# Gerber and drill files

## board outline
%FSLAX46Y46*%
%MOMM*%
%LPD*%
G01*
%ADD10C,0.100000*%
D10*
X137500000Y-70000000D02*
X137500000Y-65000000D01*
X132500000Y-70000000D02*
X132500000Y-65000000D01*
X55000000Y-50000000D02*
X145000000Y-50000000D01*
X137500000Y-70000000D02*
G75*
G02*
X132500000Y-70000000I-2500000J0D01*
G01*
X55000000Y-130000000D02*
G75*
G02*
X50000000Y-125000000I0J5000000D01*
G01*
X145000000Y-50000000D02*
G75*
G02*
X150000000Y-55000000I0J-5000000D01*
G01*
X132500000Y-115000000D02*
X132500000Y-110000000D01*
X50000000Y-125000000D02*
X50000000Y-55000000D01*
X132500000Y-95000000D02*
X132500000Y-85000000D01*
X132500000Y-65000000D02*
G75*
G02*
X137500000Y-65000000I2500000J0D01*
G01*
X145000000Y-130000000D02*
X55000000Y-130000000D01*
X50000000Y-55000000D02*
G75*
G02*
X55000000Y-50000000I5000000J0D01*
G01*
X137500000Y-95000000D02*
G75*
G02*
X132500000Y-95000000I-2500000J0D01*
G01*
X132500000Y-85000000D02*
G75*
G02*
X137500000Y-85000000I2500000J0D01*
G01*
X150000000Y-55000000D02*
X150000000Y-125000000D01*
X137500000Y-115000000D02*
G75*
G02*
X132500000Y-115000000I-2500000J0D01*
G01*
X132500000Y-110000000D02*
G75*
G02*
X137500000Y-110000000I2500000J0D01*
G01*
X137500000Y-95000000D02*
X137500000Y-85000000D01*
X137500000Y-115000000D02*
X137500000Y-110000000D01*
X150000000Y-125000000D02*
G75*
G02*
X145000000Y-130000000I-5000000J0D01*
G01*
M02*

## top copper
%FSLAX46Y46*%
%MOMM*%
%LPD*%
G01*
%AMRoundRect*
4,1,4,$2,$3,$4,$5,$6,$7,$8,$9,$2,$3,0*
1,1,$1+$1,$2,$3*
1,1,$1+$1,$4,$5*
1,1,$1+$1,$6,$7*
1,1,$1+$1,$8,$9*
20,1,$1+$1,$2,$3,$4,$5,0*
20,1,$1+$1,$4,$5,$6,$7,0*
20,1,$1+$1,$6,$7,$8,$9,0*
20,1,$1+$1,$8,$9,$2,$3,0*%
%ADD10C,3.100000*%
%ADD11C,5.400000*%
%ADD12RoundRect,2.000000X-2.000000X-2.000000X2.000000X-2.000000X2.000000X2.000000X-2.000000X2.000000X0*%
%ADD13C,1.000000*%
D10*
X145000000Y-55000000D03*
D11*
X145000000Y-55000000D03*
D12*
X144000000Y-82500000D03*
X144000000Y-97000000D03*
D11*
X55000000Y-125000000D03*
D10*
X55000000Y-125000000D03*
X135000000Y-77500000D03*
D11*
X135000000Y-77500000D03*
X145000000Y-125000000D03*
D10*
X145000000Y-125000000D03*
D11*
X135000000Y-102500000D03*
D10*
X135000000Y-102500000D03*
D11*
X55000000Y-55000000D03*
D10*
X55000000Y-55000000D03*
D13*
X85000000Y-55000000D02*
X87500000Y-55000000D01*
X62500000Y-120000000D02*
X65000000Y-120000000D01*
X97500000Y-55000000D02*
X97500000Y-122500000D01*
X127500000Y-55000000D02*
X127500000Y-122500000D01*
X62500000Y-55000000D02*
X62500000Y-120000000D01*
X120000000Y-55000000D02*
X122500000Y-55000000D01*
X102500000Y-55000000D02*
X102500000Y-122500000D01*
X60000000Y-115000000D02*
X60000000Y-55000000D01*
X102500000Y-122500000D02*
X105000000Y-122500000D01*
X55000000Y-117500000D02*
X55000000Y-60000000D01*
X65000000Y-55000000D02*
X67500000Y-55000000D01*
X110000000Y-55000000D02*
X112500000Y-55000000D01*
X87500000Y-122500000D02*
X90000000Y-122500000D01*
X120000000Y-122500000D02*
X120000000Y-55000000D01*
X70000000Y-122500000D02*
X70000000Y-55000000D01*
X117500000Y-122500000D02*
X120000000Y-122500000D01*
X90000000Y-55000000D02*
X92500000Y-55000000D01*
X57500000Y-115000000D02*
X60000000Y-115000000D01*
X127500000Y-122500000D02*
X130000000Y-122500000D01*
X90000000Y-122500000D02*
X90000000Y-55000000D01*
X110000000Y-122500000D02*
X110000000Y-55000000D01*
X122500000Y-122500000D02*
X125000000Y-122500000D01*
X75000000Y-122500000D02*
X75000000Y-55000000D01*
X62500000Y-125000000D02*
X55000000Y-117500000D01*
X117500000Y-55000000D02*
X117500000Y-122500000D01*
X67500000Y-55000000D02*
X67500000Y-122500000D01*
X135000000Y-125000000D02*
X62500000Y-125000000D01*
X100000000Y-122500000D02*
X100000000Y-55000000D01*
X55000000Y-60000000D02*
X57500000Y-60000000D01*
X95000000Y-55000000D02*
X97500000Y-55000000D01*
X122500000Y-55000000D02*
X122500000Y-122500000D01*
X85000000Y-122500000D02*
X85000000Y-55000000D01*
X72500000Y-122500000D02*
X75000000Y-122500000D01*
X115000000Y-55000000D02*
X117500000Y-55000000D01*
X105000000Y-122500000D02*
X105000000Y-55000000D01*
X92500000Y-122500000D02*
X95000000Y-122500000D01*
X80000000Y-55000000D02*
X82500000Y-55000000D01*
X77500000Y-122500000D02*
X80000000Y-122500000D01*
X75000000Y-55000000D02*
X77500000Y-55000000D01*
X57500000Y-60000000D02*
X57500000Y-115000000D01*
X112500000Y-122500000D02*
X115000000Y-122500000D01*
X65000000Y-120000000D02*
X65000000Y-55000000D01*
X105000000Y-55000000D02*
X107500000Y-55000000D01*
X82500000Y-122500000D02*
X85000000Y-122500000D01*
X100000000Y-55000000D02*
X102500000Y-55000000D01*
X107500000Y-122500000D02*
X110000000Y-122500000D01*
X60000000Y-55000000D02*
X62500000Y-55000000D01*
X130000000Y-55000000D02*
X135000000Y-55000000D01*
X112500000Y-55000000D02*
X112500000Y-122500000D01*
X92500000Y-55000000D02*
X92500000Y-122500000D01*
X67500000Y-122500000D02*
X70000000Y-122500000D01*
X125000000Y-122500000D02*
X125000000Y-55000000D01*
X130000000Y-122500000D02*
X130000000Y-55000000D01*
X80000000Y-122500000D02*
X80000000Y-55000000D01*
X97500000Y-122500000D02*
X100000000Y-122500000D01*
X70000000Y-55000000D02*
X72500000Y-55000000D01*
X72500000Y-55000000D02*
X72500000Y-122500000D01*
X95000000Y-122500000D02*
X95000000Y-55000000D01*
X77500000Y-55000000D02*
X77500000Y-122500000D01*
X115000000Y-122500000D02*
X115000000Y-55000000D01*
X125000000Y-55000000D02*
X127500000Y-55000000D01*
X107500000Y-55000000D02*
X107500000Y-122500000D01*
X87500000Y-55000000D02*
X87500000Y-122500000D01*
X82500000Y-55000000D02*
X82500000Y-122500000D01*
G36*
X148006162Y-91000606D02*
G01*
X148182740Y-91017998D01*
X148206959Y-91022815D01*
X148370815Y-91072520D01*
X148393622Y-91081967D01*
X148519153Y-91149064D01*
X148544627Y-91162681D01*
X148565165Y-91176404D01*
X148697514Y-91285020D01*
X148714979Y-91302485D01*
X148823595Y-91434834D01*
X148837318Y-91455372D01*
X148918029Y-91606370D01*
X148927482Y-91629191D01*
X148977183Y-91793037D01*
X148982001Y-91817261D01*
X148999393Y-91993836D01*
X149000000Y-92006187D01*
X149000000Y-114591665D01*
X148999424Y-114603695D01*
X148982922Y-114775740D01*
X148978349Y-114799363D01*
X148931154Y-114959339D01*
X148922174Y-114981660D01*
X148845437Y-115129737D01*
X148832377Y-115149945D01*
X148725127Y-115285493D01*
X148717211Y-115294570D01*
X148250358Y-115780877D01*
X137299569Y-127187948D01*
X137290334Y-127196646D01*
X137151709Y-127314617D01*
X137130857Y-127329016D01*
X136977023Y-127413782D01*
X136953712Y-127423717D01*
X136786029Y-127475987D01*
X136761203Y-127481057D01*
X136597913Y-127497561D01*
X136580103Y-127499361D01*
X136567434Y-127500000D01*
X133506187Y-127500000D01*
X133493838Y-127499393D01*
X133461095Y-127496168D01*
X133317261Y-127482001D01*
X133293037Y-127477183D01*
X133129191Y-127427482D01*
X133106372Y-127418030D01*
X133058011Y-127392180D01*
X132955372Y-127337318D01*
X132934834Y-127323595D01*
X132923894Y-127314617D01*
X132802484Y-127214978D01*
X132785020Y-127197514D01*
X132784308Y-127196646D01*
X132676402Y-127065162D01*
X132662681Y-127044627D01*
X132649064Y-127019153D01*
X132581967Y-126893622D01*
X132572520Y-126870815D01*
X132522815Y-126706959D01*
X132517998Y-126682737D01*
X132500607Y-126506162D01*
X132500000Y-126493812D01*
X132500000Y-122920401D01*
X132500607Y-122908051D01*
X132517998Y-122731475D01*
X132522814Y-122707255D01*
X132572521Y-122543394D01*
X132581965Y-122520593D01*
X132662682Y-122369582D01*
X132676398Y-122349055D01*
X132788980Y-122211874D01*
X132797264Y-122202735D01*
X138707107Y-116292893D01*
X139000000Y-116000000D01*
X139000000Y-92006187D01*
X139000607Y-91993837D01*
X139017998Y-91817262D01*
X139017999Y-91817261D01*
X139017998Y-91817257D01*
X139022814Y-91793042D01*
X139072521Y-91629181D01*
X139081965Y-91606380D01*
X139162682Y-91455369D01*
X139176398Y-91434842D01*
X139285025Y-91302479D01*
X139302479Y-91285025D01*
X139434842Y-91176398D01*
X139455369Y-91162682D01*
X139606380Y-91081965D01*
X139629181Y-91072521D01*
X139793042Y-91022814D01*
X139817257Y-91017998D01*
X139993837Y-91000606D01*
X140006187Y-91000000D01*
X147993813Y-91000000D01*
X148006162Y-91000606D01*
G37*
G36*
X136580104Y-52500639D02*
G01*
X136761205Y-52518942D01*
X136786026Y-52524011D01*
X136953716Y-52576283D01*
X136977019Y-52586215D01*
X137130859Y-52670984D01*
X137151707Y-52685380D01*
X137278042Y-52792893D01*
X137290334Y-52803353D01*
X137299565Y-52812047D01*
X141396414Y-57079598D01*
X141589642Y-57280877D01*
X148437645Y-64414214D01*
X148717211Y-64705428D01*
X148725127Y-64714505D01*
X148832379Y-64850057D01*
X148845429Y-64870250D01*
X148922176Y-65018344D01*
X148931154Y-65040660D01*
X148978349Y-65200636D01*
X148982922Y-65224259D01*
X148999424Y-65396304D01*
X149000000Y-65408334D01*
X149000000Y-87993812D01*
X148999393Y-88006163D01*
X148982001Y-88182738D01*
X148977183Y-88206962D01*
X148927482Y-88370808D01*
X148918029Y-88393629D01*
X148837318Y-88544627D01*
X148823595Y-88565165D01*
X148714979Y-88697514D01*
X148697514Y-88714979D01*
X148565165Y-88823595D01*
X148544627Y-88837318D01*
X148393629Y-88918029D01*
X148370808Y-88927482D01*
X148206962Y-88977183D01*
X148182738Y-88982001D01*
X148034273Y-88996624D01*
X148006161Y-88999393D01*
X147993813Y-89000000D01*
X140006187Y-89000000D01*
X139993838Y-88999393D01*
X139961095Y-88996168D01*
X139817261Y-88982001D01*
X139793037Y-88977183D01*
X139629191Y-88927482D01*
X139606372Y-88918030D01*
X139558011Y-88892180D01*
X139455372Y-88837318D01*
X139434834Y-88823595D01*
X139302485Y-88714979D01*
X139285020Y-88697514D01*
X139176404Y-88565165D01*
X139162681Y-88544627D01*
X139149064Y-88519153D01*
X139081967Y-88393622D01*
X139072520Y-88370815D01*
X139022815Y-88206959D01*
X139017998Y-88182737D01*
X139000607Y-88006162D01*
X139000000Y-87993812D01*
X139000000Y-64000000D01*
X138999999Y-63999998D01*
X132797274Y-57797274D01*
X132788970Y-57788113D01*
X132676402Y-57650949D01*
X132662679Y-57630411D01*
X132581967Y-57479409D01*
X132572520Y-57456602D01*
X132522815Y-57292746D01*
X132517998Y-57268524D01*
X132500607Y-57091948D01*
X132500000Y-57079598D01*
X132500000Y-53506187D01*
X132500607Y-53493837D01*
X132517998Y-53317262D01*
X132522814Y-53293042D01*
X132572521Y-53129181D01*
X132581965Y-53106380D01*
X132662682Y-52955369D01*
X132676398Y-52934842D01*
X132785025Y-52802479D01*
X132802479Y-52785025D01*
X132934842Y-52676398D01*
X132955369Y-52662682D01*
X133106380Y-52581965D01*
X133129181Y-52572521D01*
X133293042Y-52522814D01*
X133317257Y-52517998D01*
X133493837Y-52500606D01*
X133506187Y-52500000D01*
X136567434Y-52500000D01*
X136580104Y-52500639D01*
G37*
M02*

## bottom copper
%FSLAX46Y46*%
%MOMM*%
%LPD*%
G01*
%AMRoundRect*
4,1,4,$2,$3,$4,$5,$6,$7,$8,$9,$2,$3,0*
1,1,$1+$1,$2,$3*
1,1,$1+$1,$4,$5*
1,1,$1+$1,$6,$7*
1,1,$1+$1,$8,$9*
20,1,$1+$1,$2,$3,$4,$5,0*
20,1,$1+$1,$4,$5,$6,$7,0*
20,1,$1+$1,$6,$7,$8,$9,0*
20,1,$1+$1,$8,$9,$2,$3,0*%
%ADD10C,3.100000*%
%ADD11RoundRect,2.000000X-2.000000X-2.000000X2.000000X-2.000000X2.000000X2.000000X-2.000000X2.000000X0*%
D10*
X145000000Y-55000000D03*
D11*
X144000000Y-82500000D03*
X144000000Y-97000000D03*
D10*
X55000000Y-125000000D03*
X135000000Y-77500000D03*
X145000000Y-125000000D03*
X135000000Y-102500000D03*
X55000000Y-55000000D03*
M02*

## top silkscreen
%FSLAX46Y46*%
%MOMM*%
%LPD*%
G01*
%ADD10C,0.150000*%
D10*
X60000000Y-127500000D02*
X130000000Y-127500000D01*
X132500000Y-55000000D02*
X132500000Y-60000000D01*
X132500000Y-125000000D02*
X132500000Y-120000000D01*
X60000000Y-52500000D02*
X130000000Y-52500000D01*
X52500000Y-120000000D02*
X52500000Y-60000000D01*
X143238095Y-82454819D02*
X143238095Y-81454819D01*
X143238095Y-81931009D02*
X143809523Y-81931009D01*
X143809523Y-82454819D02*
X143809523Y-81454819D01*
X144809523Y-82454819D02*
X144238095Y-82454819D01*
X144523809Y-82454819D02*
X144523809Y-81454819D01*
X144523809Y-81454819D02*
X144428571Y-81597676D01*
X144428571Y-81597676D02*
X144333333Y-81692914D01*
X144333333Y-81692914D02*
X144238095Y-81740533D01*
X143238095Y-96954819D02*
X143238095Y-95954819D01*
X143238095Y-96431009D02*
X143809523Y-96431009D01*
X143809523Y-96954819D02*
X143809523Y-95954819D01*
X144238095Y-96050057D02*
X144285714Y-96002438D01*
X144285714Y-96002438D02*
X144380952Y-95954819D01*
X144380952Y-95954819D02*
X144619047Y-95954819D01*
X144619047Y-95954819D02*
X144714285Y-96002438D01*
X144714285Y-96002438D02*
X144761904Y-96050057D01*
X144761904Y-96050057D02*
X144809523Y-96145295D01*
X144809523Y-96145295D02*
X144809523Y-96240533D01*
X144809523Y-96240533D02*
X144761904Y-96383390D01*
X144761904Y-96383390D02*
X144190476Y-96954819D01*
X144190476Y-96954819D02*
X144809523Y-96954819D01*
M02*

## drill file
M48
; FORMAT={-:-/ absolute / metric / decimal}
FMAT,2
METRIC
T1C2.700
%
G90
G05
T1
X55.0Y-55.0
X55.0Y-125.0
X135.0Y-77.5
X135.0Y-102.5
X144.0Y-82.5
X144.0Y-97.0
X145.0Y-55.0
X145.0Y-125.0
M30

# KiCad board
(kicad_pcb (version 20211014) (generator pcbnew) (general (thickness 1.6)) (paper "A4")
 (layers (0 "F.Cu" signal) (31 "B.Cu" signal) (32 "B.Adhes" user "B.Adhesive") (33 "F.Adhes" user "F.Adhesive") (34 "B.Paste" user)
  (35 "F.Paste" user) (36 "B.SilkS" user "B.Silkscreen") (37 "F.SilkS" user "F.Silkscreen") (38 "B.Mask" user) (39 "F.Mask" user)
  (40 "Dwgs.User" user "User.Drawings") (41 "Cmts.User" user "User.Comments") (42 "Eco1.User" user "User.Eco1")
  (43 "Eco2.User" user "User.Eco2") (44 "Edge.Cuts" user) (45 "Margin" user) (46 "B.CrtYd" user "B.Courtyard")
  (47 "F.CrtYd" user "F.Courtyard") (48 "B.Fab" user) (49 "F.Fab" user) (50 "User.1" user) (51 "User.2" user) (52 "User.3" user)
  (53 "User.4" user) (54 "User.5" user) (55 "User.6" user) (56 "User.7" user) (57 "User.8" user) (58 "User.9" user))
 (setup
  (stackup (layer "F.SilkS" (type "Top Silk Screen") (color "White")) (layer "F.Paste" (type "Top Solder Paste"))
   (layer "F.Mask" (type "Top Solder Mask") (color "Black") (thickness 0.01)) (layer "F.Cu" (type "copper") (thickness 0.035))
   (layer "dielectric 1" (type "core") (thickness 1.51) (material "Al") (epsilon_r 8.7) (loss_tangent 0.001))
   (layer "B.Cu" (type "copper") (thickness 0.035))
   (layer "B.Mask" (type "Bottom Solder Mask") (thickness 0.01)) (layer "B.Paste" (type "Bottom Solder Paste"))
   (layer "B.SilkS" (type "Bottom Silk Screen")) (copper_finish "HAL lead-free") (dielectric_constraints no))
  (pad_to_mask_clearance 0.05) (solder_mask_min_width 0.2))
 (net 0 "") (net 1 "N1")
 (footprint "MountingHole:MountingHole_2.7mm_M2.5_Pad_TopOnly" (layer "F.Cu") (at 145 55)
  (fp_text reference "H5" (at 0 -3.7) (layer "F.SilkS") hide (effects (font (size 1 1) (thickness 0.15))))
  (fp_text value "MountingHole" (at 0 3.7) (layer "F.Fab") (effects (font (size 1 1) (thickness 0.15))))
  (pad "1" thru_hole circle (at 0 0) (size 3.1 3.1) (drill 2.7) (layers *.Cu *.Mask))
  (pad "1" connect circle (at 0 0) (size 5.4 5.4) (layers "F.Cu" "F.Mask")))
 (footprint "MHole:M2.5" (layer "F.Cu") (at 144 82.5)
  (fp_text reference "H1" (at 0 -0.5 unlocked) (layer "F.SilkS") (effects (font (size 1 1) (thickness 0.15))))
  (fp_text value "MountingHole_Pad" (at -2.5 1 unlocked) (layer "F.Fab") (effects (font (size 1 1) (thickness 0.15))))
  (pad "1" thru_hole roundrect (at 0 0) (size 8 8) (drill 2.7) (layers *.Cu *.Mask) (roundrect_rratio 0.25) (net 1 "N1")))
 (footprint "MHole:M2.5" (layer "F.Cu") (at 144 97)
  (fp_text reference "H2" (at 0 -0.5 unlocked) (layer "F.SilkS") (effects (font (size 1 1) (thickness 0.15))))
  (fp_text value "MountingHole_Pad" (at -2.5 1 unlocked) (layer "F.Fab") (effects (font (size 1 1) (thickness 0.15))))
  (pad "1" thru_hole roundrect (at 0 0) (size 8 8) (drill 2.7) (layers *.Cu *.Mask) (roundrect_rratio 0.25) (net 1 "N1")))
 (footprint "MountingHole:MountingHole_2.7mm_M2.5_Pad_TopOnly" (layer "F.Cu") (at 55 125)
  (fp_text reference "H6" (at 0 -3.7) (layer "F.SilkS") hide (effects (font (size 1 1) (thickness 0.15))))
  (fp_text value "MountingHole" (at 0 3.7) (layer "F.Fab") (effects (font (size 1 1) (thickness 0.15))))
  (pad "1" connect circle (at 0 0) (size 5.4 5.4) (layers "F.Cu" "F.Mask"))
  (pad "1" thru_hole circle (at 0 0) (size 3.1 3.1) (drill 2.7) (layers *.Cu *.Mask)))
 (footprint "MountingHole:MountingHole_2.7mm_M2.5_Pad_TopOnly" (layer "F.Cu") (at 135 77.5)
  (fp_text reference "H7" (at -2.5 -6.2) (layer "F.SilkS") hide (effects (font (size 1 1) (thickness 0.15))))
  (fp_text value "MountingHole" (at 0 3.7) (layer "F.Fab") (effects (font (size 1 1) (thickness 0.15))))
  (pad "1" thru_hole circle (at 0 0) (size 3.1 3.1) (drill 2.7) (layers *.Cu *.Mask))
  (pad "1" connect circle (at 0 0) (size 5.4 5.4) (layers "F.Cu" "F.Mask")))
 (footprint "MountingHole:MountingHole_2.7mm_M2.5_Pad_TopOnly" (layer "F.Cu") (at 145 125)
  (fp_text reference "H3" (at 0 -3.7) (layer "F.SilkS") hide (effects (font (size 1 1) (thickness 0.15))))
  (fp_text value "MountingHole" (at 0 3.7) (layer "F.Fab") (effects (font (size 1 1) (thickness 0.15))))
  (pad "1" connect circle (at 0 0) (size 5.4 5.4) (layers "F.Cu" "F.Mask"))
  (pad "1" thru_hole circle (at 0 0) (size 3.1 3.1) (drill 2.7) (layers *.Cu *.Mask)))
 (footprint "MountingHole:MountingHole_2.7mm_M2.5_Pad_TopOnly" (layer "F.Cu") (at 135 102.5)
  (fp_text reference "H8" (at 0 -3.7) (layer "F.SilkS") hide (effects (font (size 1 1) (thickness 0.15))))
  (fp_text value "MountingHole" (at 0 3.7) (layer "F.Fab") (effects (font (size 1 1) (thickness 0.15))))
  (pad "1" connect circle (at 0 0) (size 5.4 5.4) (layers "F.Cu" "F.Mask"))
  (pad "1" thru_hole circle (at 0 0) (size 3.1 3.1) (drill 2.7) (layers *.Cu *.Mask)))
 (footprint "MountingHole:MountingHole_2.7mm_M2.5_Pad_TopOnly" (layer "F.Cu") (at 55 55)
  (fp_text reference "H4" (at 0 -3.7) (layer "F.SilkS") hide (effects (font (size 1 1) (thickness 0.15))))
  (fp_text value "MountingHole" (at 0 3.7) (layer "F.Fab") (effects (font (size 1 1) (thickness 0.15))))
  (pad "1" connect circle (at 0 0) (size 5.4 5.4) (layers "F.Cu" "F.Mask"))
  (pad "1" thru_hole circle (at 0 0) (size 3.1 3.1) (drill 2.7) (layers *.Cu *.Mask)))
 (gr_line (start 60 127.5) (end 130 127.5) (layer "F.SilkS") (width 0.15))
 (gr_line (start 132.5 55) (end 132.5 60) (layer "F.SilkS") (width 0.15))
 (gr_line (start 132.5 125) (end 132.5 120) (layer "F.SilkS") (width 0.15))
 (gr_line (start 60 52.5) (end 130 52.5) (layer "F.SilkS") (width 0.15))
 (gr_line (start 52.5 120) (end 52.5 60) (layer "F.SilkS") (width 0.15))
 (gr_line (start 137.5 70) (end 137.5 65) (layer "Edge.Cuts") (width 0.1))
 (gr_line (start 132.5 70) (end 132.5 65) (layer "Edge.Cuts") (width 0.1))
 (gr_line (start 55 50) (end 145 50) (layer "Edge.Cuts") (width 0.1))
 (gr_arc (start 137.5 70) (mid 135 72.5) (end 132.5 70) (layer "Edge.Cuts") (width 0.1))
 (gr_arc (start 55 130) (mid 51.464466 128.535534) (end 50 125) (layer "Edge.Cuts") (width 0.1))
 (gr_arc (start 145 50) (mid 148.535534 51.464466) (end 150 55) (layer "Edge.Cuts") (width 0.1))
 (gr_line (start 132.5 115) (end 132.5 110) (layer "Edge.Cuts") (width 0.1))
 (gr_line (start 50 125) (end 50 55) (layer "Edge.Cuts") (width 0.1))
 (gr_line (start 132.5 95) (end 132.5 85) (layer "Edge.Cuts") (width 0.1))
 (gr_arc (start 132.5 65) (mid 135 62.5) (end 137.5 65) (layer "Edge.Cuts") (width 0.1))
 (gr_line (start 145 130) (end 55 130) (layer "Edge.Cuts") (width 0.1))
 (gr_arc (start 50 55) (mid 51.464466 51.464466) (end 55 50) (layer "Edge.Cuts") (width 0.1))
 (gr_arc (start 137.5 95) (mid 135 97.5) (end 132.5 95) (layer "Edge.Cuts") (width 0.1))
 (gr_arc (start 132.5 85) (mid 135 82.5) (end 137.5 85) (layer "Edge.Cuts") (width 0.1))
 (gr_line (start 150 55) (end 150 125) (layer "Edge.Cuts") (width 0.1))
 (gr_arc (start 137.5 115) (mid 135 117.5) (end 132.5 115) (layer "Edge.Cuts") (width 0.1))
 (gr_arc (start 132.5 110) (mid 135 107.5) (end 137.5 110) (layer "Edge.Cuts") (width 0.1))
 (gr_line (start 137.5 95) (end 137.5 85) (layer "Edge.Cuts") (width 0.1))
 (gr_line (start 137.5 115) (end 137.5 110) (layer "Edge.Cuts") (width 0.1))
 (gr_arc (start 150 125) (mid 148.535534 128.535534) (end 145 130) (layer "Edge.Cuts") (width 0.1))
 (segment (start 85 55) (end 87.5 55) (width 1) (layer "F.Cu") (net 1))
 (segment (start 62.5 120) (end 65 120) (width 1) (layer "F.Cu") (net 1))
 (segment (start 97.5 55) (end 97.5 122.5) (width 1) (layer "F.Cu") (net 1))
 (segment (start 127.5 55) (end 127.5 122.5) (width 1) (layer "F.Cu") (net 1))
 (segment (start 62.5 55) (end 62.5 120) (width 1) (layer "F.Cu") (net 1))
 (segment (start 120 55) (end 122.5 55) (width 1) (layer "F.Cu") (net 1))
 (segment (start 102.5 55) (end 102.5 122.5) (width 1) (layer "F.Cu") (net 1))
 (segment (start 60 115) (end 60 55) (width 1) (layer "F.Cu") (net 1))
 (segment (start 102.5 122.5) (end 105 122.5) (width 1) (layer "F.Cu") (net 1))
 (segment (start 55 117.5) (end 55 60) (width 1) (layer "F.Cu") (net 1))
 (segment (start 65 55) (end 67.5 55) (width 1) (layer "F.Cu") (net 1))
 (segment (start 110 55) (end 112.5 55) (width 1) (layer "F.Cu") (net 1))
 (segment (start 87.5 122.5) (end 90 122.5) (width 1) (layer "F.Cu") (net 1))
 (segment (start 120 122.5) (end 120 55) (width 1) (layer "F.Cu") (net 1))
 (segment (start 70 122.5) (end 70 55) (width 1) (layer "F.Cu") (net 1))
 (segment (start 117.5 122.5) (end 120 122.5) (width 1) (layer "F.Cu") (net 1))
 (segment (start 90 55) (end 92.5 55) (width 1) (layer "F.Cu") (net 1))
 (segment (start 57.5 115) (end 60 115) (width 1) (layer "F.Cu") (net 1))
 (segment (start 127.5 122.5) (end 130 122.5) (width 1) (layer "F.Cu") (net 1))
 (segment (start 90 122.5) (end 90 55) (width 1) (layer "F.Cu") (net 1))
 (segment (start 110 122.5) (end 110 55) (width 1) (layer "F.Cu") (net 1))
 (segment (start 122.5 122.5) (end 125 122.5) (width 1) (layer "F.Cu") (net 1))
 (segment (start 75 122.5) (end 75 55) (width 1) (layer "F.Cu") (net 1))
 (segment (start 62.5 125) (end 55 117.5) (width 1) (layer "F.Cu") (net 1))
 (segment (start 117.5 55) (end 117.5 122.5) (width 1) (layer "F.Cu") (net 1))
 (segment (start 67.5 55) (end 67.5 122.5) (width 1) (layer "F.Cu") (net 1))
 (segment (start 135 125) (end 62.5 125) (width 1) (layer "F.Cu") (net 1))
 (segment (start 100 122.5) (end 100 55) (width 1) (layer "F.Cu") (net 1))
 (segment (start 55 60) (end 57.5 60) (width 1) (layer "F.Cu") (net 1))
 (segment (start 95 55) (end 97.5 55) (width 1) (layer "F.Cu") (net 1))
 (segment (start 122.5 55) (end 122.5 122.5) (width 1) (layer "F.Cu") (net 1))
 (segment (start 85 122.5) (end 85 55) (width 1) (layer "F.Cu") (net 1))
 (segment (start 72.5 122.5) (end 75 122.5) (width 1) (layer "F.Cu") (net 1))
 (segment (start 115 55) (end 117.5 55) (width 1) (layer "F.Cu") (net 1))
 (segment (start 105 122.5) (end 105 55) (width 1) (layer "F.Cu") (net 1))
 (segment (start 92.5 122.5) (end 95 122.5) (width 1) (layer "F.Cu") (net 1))
 (segment (start 80 55) (end 82.5 55) (width 1) (layer "F.Cu") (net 1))
 (segment (start 77.5 122.5) (end 80 122.5) (width 1) (layer "F.Cu") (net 1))
 (segment (start 75 55) (end 77.5 55) (width 1) (layer "F.Cu") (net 1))
 (segment (start 57.5 60) (end 57.5 115) (width 1) (layer "F.Cu") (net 1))
 (segment (start 112.5 122.5) (end 115 122.5) (width 1) (layer "F.Cu") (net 1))
 (segment (start 65 120) (end 65 55) (width 1) (layer "F.Cu") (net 1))
 (segment (start 105 55) (end 107.5 55) (width 1) (layer "F.Cu") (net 1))
 (segment (start 82.5 122.5) (end 85 122.5) (width 1) (layer "F.Cu") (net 1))
 (segment (start 100 55) (end 102.5 55) (width 1) (layer "F.Cu") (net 1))
 (segment (start 107.5 122.5) (end 110 122.5) (width 1) (layer "F.Cu") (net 1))
 (segment (start 60 55) (end 62.5 55) (width 1) (layer "F.Cu") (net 1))
 (segment (start 130 55) (end 135 55) (width 1) (layer "F.Cu") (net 1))
 (segment (start 112.5 55) (end 112.5 122.5) (width 1) (layer "F.Cu") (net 1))
 (segment (start 92.5 55) (end 92.5 122.5) (width 1) (layer "F.Cu") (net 1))
 (segment (start 67.5 122.5) (end 70 122.5) (width 1) (layer "F.Cu") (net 1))
 (segment (start 125 122.5) (end 125 55) (width 1) (layer "F.Cu") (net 1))
 (segment (start 130 122.5) (end 130 55) (width 1) (layer "F.Cu") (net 1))
 (segment (start 80 122.5) (end 80 55) (width 1) (layer "F.Cu") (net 1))
 (segment (start 97.5 122.5) (end 100 122.5) (width 1) (layer "F.Cu") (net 1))
 (segment (start 70 55) (end 72.5 55) (width 1) (layer "F.Cu") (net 1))
 (segment (start 72.5 55) (end 72.5 122.5) (width 1) (layer "F.Cu") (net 1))
 (segment (start 95 122.5) (end 95 55) (width 1) (layer "F.Cu") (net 1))
 (segment (start 77.5 55) (end 77.5 122.5) (width 1) (layer "F.Cu") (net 1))
 (segment (start 115 122.5) (end 115 55) (width 1) (layer "F.Cu") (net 1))
 (segment (start 125 55) (end 127.5 55) (width 1) (layer "F.Cu") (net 1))
 (segment (start 107.5 55) (end 107.5 122.5) (width 1) (layer "F.Cu") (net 1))
 (segment (start 87.5 55) (end 87.5 122.5) (width 1) (layer "F.Cu") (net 1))
 (segment (start 82.5 55) (end 82.5 122.5) (width 1) (layer "F.Cu") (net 1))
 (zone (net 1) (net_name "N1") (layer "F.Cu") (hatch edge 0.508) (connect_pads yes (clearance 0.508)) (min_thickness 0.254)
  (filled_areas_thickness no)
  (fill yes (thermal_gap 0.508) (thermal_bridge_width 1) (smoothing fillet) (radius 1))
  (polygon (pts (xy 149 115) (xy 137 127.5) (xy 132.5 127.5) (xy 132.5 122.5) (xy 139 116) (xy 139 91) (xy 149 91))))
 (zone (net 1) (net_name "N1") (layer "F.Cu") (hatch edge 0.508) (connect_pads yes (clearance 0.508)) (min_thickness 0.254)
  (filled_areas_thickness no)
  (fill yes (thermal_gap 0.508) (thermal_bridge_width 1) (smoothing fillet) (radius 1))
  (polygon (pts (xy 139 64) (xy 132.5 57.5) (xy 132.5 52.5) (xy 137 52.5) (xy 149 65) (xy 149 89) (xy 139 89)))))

